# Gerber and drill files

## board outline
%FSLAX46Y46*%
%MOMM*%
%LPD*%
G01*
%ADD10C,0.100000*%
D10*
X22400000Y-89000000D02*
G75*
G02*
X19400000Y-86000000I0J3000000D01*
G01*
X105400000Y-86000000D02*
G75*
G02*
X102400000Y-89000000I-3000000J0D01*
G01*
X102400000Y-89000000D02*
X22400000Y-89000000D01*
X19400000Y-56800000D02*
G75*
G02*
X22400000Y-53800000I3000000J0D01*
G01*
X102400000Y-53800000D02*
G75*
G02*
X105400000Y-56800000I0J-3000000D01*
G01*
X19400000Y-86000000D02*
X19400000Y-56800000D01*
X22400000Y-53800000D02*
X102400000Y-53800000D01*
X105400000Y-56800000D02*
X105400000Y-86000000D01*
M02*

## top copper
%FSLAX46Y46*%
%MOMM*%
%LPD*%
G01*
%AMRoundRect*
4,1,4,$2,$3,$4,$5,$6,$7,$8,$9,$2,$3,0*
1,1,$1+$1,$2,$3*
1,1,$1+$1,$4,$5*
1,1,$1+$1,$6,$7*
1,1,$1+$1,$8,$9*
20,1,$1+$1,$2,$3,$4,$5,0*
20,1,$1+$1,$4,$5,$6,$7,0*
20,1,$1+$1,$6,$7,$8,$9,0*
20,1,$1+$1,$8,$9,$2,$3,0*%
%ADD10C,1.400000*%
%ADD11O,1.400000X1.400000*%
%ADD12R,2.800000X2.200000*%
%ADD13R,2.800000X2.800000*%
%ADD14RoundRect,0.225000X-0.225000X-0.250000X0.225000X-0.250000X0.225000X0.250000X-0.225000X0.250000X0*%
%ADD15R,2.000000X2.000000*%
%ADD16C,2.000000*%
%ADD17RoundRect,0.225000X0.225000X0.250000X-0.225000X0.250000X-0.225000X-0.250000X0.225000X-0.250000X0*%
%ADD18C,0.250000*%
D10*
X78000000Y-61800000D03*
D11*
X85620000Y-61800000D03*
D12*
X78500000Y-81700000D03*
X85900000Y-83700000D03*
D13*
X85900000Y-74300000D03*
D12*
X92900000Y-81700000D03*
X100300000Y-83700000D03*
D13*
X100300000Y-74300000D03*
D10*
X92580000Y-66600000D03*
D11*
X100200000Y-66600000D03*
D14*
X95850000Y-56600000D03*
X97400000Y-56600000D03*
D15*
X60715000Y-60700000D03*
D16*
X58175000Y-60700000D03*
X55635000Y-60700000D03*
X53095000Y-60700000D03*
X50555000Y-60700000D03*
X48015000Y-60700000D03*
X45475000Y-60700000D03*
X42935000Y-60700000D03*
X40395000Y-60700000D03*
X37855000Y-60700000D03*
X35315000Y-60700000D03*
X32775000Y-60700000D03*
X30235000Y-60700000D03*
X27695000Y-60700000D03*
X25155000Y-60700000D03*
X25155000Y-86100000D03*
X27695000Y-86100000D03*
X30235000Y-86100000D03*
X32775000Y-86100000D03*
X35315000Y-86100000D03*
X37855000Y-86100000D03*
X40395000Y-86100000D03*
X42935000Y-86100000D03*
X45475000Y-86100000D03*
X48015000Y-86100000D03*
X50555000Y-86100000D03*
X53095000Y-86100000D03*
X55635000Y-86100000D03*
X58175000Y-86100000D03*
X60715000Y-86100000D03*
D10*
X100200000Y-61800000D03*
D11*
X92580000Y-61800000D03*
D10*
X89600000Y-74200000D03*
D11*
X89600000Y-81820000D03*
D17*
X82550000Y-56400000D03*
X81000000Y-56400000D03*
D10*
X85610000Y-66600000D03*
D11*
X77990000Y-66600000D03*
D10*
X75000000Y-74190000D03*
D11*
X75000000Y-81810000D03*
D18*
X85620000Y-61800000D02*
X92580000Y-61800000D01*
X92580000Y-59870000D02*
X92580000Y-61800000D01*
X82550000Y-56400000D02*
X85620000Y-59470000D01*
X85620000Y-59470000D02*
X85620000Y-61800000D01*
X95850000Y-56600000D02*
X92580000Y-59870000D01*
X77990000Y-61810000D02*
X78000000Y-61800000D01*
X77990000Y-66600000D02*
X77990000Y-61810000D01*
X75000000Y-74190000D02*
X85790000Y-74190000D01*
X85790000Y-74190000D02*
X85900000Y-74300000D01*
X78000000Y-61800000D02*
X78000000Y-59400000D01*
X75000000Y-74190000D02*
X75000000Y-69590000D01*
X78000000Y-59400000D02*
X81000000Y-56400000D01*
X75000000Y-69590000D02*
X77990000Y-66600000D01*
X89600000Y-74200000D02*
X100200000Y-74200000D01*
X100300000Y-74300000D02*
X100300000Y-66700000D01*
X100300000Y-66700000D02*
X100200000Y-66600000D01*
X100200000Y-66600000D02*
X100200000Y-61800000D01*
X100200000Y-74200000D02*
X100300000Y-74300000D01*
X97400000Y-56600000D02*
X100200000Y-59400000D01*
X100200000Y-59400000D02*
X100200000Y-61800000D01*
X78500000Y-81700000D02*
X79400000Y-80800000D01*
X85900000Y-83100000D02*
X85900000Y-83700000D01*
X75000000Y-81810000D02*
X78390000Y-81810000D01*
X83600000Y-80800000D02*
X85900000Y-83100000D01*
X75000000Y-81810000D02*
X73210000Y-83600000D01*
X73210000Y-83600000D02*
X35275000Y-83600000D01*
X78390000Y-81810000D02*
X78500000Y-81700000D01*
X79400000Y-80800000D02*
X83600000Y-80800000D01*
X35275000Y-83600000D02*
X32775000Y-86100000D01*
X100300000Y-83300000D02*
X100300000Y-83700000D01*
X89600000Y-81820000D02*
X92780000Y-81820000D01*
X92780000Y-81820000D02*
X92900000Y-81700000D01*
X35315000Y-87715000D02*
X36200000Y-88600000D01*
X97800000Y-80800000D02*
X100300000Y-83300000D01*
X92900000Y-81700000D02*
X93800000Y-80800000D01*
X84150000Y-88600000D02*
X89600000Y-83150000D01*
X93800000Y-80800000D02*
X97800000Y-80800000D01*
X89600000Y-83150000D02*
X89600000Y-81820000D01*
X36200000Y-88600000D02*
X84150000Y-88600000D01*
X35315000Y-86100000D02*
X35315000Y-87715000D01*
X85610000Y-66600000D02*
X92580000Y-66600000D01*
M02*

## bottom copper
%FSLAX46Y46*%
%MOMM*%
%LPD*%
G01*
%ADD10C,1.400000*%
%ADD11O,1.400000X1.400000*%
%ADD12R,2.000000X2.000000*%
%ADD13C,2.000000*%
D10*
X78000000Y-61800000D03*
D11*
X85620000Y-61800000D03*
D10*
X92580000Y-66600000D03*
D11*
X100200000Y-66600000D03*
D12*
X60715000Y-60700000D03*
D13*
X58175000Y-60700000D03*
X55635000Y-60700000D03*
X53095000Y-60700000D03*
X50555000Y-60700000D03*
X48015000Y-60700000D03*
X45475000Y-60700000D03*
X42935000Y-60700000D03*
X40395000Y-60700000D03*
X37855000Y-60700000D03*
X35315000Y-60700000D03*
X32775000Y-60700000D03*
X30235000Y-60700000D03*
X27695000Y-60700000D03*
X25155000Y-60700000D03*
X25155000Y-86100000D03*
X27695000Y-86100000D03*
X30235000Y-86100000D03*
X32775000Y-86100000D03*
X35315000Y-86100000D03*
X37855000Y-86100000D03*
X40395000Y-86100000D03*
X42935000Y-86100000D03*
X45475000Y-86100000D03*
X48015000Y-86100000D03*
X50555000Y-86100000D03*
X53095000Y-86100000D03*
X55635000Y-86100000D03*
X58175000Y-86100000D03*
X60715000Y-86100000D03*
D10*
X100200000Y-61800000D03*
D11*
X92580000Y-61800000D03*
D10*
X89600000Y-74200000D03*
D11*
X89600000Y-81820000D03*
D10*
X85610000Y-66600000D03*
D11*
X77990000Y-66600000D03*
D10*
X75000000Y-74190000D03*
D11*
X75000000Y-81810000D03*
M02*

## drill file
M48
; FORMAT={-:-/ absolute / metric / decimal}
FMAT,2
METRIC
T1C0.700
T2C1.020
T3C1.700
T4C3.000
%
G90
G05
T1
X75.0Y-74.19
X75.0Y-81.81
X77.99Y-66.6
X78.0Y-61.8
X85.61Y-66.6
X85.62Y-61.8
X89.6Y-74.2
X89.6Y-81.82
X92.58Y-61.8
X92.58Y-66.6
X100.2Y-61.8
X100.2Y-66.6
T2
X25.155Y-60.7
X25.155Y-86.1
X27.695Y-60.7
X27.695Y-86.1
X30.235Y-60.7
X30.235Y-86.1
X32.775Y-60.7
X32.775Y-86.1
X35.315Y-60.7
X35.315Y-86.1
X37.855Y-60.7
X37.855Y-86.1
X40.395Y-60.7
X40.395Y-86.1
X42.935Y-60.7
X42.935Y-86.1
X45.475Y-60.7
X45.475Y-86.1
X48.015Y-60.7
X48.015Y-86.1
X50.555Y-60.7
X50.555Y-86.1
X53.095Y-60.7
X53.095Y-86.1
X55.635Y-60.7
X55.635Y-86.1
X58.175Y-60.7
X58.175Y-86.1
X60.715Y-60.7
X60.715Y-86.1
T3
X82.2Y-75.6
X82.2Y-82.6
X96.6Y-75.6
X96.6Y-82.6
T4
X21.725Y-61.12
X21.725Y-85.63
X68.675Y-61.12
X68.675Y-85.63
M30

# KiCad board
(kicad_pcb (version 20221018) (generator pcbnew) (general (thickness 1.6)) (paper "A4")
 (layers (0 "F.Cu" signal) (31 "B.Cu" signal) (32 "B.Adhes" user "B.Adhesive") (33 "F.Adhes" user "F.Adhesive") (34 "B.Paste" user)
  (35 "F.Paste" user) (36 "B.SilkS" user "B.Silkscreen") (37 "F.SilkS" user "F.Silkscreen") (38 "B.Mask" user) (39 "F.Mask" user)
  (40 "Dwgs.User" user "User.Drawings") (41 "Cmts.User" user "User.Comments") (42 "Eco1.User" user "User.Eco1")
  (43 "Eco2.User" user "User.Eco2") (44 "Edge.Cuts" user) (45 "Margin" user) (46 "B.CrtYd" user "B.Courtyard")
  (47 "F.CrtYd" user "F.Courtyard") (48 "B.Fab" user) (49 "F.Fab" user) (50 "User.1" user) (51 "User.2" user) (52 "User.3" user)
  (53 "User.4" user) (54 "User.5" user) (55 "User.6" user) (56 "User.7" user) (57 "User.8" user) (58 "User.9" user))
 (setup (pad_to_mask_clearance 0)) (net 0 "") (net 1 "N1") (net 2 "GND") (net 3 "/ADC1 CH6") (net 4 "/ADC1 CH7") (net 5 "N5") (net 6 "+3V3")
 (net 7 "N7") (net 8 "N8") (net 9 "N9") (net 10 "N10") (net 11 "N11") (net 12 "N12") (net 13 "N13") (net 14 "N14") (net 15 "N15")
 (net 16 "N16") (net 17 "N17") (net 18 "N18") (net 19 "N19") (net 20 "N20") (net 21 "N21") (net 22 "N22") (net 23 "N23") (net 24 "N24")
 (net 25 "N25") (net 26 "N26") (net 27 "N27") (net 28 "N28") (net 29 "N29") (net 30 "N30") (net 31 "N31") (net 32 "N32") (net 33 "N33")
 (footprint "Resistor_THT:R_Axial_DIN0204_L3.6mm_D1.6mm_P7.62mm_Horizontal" (layer "F.Cu") (at 78 61.8)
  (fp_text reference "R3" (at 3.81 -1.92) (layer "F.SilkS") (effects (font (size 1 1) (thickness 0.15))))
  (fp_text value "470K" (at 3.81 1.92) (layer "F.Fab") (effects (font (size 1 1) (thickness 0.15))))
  (pad "1" thru_hole circle (at 0 0) (size 1.4 1.4) (drill 0.7) (layers "*.Cu" "*.Mask") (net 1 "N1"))
  (pad "2" thru_hole oval (at 7.62 0) (size 1.4 1.4) (drill 0.7) (layers "*.Cu" "*.Mask") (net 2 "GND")))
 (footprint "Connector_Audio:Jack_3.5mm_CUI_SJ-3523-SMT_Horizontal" (layer "F.Cu") (at 82.2 80.1 180)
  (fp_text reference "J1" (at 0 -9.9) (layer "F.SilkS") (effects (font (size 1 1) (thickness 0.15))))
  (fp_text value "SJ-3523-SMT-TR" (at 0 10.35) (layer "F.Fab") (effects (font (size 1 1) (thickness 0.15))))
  (pad "" np_thru_hole circle (at 0 -2.5 180) (size 1.7 1.7) (drill 1.7) (layers "*.Cu" "*.Mask"))
  (pad "" np_thru_hole circle (at 0 4.5 180) (size 1.7 1.7) (drill 1.7) (layers "*.Cu" "*.Mask"))
  (pad "R" smd rect (at 3.7 -1.6 180) (size 2.8 2.2) (layers "F.Cu" "F.Paste" "F.Mask") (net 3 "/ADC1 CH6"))
  (pad "S" smd rect (at -3.7 -3.6 180) (size 2.8 2.2) (layers "F.Cu" "F.Paste" "F.Mask") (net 3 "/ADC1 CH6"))
  (pad "T" smd rect (at -3.7 5.8 180) (size 2.8 2.8) (layers "F.Cu" "F.Paste" "F.Mask") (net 1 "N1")))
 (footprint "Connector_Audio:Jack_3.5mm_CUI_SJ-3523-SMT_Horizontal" (layer "F.Cu") (at 96.6 80.1 180)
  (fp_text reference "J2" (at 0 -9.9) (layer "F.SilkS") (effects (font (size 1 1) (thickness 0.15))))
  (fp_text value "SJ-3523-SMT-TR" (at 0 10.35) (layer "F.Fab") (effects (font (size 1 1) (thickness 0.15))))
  (pad "" np_thru_hole circle (at 0 -2.5 180) (size 1.7 1.7) (drill 1.7) (layers "*.Cu" "*.Mask"))
  (pad "" np_thru_hole circle (at 0 4.5 180) (size 1.7 1.7) (drill 1.7) (layers "*.Cu" "*.Mask"))
  (pad "R" smd rect (at 3.7 -1.6 180) (size 2.8 2.2) (layers "F.Cu" "F.Paste" "F.Mask") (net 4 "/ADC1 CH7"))
  (pad "S" smd rect (at -3.7 -3.6 180) (size 2.8 2.2) (layers "F.Cu" "F.Paste" "F.Mask") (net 4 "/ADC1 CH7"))
  (pad "T" smd rect (at -3.7 5.8 180) (size 2.8 2.8) (layers "F.Cu" "F.Paste" "F.Mask") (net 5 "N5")))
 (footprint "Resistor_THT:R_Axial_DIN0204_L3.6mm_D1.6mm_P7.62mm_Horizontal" (layer "F.Cu") (at 92.58 66.6)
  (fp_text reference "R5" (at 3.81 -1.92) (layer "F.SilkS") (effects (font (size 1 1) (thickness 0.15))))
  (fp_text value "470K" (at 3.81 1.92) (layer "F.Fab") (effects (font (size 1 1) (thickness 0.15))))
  (pad "1" thru_hole circle (at 0 0) (size 1.4 1.4) (drill 0.7) (layers "*.Cu" "*.Mask") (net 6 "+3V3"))
  (pad "2" thru_hole oval (at 7.62 0) (size 1.4 1.4) (drill 0.7) (layers "*.Cu" "*.Mask") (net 5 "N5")))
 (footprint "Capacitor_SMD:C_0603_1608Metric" (layer "F.Cu") (at 96.625 56.6)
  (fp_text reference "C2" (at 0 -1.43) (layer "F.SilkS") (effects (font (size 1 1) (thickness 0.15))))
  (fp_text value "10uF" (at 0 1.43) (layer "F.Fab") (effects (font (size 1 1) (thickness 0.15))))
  (pad "1" smd roundrect (at -0.775 0) (size 0.9 0.95) (layers "F.Cu" "F.Paste" "F.Mask") (roundrect_rratio 0.25) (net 2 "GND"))
  (pad "2" smd roundrect (at 0.775 0) (size 0.9 0.95) (layers "F.Cu" "F.Paste" "F.Mask") (roundrect_rratio 0.25) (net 5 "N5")))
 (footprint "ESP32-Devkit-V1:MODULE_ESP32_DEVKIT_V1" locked (layer "F.Cu") (at 45.2 73.4 -90)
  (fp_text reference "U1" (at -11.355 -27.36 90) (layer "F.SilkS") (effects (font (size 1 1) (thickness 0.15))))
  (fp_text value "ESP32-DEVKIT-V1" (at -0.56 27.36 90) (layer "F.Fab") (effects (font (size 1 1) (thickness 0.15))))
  (pad "" np_thru_hole circle locked (at -12.28 -23.475 270) (size 3 3) (drill 3) (layers "*.Cu" "*.Mask"))
  (pad "" np_thru_hole circle locked (at -12.28 23.475 270) (size 3 3) (drill 3) (layers "*.Cu" "*.Mask"))
  (pad "" np_thru_hole circle locked (at 12.23 -23.475 270) (size 3 3) (drill 3) (layers "*.Cu" "*.Mask"))
  (pad "" np_thru_hole circle locked (at 12.23 23.475 270) (size 3 3) (drill 3) (layers "*.Cu" "*.Mask"))
  (pad "1" thru_hole rect locked (at -12.7 -15.515 270) (size 2 2) (drill 1.02) (layers "*.Cu" "*.Mask") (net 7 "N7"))
  (pad "2" thru_hole circle locked (at -12.7 -12.975 270) (size 2 2) (drill 1.02) (layers "*.Cu" "*.Mask") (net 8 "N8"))
  (pad "3" thru_hole circle locked (at -12.7 -10.435 270) (size 2 2) (drill 1.02) (layers "*.Cu" "*.Mask") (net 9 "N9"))
  (pad "4" thru_hole circle locked (at -12.7 -7.895 270) (size 2 2) (drill 1.02) (layers "*.Cu" "*.Mask") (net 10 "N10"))
  (pad "5" thru_hole circle locked (at -12.7 -5.355 270) (size 2 2) (drill 1.02) (layers "*.Cu" "*.Mask") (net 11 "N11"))
  (pad "6" thru_hole circle locked (at -12.7 -2.815 270) (size 2 2) (drill 1.02) (layers "*.Cu" "*.Mask") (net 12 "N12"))
  (pad "7" thru_hole circle locked (at -12.7 -0.275 270) (size 2 2) (drill 1.02) (layers "*.Cu" "*.Mask") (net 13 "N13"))
  (pad "8" thru_hole circle locked (at -12.7 2.265 270) (size 2 2) (drill 1.02) (layers "*.Cu" "*.Mask") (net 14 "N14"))
  (pad "9" thru_hole circle locked (at -12.7 4.805 270) (size 2 2) (drill 1.02) (layers "*.Cu" "*.Mask") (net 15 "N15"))
  (pad "10" thru_hole circle locked (at -12.7 7.345 270) (size 2 2) (drill 1.02) (layers "*.Cu" "*.Mask") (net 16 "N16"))
  (pad "11" thru_hole circle locked (at -12.7 9.885 270) (size 2 2) (drill 1.02) (layers "*.Cu" "*.Mask") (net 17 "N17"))
  (pad "12" thru_hole circle locked (at -12.7 12.425 270) (size 2 2) (drill 1.02) (layers "*.Cu" "*.Mask") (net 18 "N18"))
  (pad "13" thru_hole circle locked (at -12.7 14.965 270) (size 2 2) (drill 1.02) (layers "*.Cu" "*.Mask") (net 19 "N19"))
  (pad "14" thru_hole circle locked (at -12.7 17.505 270) (size 2 2) (drill 1.02) (layers "*.Cu" "*.Mask") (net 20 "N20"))
  (pad "15" thru_hole circle locked (at -12.7 20.045 270) (size 2 2) (drill 1.02) (layers "*.Cu" "*.Mask") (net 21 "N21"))
  (pad "16" thru_hole circle locked (at 12.7 20.045 270) (size 2 2) (drill 1.02) (layers "*.Cu" "*.Mask") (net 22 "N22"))
  (pad "17" thru_hole circle locked (at 12.7 17.505 270) (size 2 2) (drill 1.02) (layers "*.Cu" "*.Mask") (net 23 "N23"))
  (pad "18" thru_hole circle locked (at 12.7 14.965 270) (size 2 2) (drill 1.02) (layers "*.Cu" "*.Mask") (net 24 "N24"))
  (pad "19" thru_hole circle locked (at 12.7 12.425 270) (size 2 2) (drill 1.02) (layers "*.Cu" "*.Mask") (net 3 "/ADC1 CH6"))
  (pad "20" thru_hole circle locked (at 12.7 9.885 270) (size 2 2) (drill 1.02) (layers "*.Cu" "*.Mask") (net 4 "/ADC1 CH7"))
  (pad "21" thru_hole circle locked (at 12.7 7.345 270) (size 2 2) (drill 1.02) (layers "*.Cu" "*.Mask") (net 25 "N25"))
  (pad "22" thru_hole circle locked (at 12.7 4.805 270) (size 2 2) (drill 1.02) (layers "*.Cu" "*.Mask") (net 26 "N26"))
  (pad "23" thru_hole circle locked (at 12.7 2.265 270) (size 2 2) (drill 1.02) (layers "*.Cu" "*.Mask") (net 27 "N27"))
  (pad "24" thru_hole circle locked (at 12.7 -0.275 270) (size 2 2) (drill 1.02) (layers "*.Cu" "*.Mask") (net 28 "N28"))
  (pad "25" thru_hole circle locked (at 12.7 -2.815 270) (size 2 2) (drill 1.02) (layers "*.Cu" "*.Mask") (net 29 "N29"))
  (pad "26" thru_hole circle locked (at 12.7 -5.355 270) (size 2 2) (drill 1.02) (layers "*.Cu" "*.Mask") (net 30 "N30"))
  (pad "27" thru_hole circle locked (at 12.7 -7.895 270) (size 2 2) (drill 1.02) (layers "*.Cu" "*.Mask") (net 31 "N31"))
  (pad "28" thru_hole circle locked (at 12.7 -10.435 270) (size 2 2) (drill 1.02) (layers "*.Cu" "*.Mask") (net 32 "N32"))
  (pad "29" thru_hole circle locked (at 12.7 -12.975 270) (size 2 2) (drill 1.02) (layers "*.Cu" "*.Mask") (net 8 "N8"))
  (pad "30" thru_hole circle locked (at 12.7 -15.515 270) (size 2 2) (drill 1.02) (layers "*.Cu" "*.Mask") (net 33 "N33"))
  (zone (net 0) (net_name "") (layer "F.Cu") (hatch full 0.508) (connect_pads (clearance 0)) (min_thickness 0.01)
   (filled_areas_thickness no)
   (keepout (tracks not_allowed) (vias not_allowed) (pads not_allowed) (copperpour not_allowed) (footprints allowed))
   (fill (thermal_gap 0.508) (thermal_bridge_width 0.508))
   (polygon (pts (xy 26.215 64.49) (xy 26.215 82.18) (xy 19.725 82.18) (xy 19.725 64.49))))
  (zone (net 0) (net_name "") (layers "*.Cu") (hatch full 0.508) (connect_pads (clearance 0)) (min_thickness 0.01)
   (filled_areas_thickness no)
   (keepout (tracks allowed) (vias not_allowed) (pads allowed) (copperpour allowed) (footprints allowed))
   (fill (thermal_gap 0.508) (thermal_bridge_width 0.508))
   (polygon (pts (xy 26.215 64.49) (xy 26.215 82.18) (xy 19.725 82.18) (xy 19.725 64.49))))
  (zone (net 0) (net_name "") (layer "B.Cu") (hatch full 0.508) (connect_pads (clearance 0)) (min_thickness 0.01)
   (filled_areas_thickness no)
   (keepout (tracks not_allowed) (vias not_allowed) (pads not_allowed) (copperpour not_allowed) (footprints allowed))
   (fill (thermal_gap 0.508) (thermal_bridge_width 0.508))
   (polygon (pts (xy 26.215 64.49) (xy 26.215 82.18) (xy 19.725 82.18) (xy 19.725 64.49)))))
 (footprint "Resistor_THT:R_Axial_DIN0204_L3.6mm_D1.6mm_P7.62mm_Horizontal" (layer "F.Cu") (at 100.2 61.8 180)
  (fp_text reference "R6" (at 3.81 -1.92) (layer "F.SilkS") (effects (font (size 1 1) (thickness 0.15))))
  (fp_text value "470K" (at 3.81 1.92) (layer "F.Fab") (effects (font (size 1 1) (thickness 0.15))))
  (pad "1" thru_hole circle (at 0 0 180) (size 1.4 1.4) (drill 0.7) (layers "*.Cu" "*.Mask") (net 5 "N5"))
  (pad "2" thru_hole oval (at 7.62 0 180) (size 1.4 1.4) (drill 0.7) (layers "*.Cu" "*.Mask") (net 2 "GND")))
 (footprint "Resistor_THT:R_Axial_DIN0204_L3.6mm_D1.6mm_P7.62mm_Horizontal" (layer "F.Cu") (at 89.6 74.2 -90)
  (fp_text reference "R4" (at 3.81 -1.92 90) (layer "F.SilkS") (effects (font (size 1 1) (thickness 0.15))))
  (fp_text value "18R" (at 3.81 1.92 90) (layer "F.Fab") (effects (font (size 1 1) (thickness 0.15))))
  (pad "1" thru_hole circle (at 0 0 270) (size 1.4 1.4) (drill 0.7) (layers "*.Cu" "*.Mask") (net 5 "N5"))
  (pad "2" thru_hole oval (at 7.62 0 270) (size 1.4 1.4) (drill 0.7) (layers "*.Cu" "*.Mask") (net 4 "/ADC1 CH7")))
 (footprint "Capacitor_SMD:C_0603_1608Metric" (layer "F.Cu") (at 81.775 56.4 180)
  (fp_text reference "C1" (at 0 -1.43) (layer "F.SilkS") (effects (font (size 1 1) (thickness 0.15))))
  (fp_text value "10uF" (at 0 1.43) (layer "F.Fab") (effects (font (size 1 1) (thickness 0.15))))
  (pad "1" smd roundrect (at -0.775 0 180) (size 0.9 0.95) (layers "F.Cu" "F.Paste" "F.Mask") (roundrect_rratio 0.25) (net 2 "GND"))
  (pad "2" smd roundrect (at 0.775 0 180) (size 0.9 0.95) (layers "F.Cu" "F.Paste" "F.Mask") (roundrect_rratio 0.25) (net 1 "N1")))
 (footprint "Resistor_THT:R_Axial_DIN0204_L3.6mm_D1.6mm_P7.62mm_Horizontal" (layer "F.Cu") (at 85.61 66.6 180)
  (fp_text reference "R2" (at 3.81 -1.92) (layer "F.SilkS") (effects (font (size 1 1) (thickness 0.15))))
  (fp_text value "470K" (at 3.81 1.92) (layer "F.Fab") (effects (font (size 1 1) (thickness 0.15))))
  (pad "1" thru_hole circle (at 0 0 180) (size 1.4 1.4) (drill 0.7) (layers "*.Cu" "*.Mask") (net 6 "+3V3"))
  (pad "2" thru_hole oval (at 7.62 0 180) (size 1.4 1.4) (drill 0.7) (layers "*.Cu" "*.Mask") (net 1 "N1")))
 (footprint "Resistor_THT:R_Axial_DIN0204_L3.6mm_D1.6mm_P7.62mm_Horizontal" (layer "F.Cu") (at 75 74.19 -90)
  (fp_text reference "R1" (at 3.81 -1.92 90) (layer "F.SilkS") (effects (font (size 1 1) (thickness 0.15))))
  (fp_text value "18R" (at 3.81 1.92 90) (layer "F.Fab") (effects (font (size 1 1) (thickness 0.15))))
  (pad "1" thru_hole circle (at 0 0 270) (size 1.4 1.4) (drill 0.7) (layers "*.Cu" "*.Mask") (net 1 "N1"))
  (pad "2" thru_hole oval (at 7.62 0 270) (size 1.4 1.4) (drill 0.7) (layers "*.Cu" "*.Mask") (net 3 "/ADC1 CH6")))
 (gr_arc (start 22.4 89) (mid 20.27868 88.12132) (end 19.4 86) (stroke (width 0.1) (type default)) (layer "Edge.Cuts"))
 (gr_arc (start 105.4 86) (mid 104.52132 88.12132) (end 102.4 89) (stroke (width 0.1) (type default)) (layer "Edge.Cuts"))
 (gr_line (start 102.4 89) (end 22.4 89) (stroke (width 0.1) (type default)) (layer "Edge.Cuts"))
 (gr_arc (start 19.4 56.8) (mid 20.27868 54.67868) (end 22.4 53.8) (stroke (width 0.1) (type default)) (layer "Edge.Cuts"))
 (gr_arc (start 102.4 53.8) (mid 104.52132 54.67868) (end 105.4 56.8) (stroke (width 0.1) (type default)) (layer "Edge.Cuts"))
 (gr_line (start 19.4 86) (end 19.4 56.8) (stroke (width 0.1) (type default)) (layer "Edge.Cuts"))
 (gr_line (start 22.4 53.8) (end 102.4 53.8) (stroke (width 0.1) (type default)) (layer "Edge.Cuts"))
 (gr_line (start 105.4 56.8) (end 105.4 86) (stroke (width 0.1) (type default)) (layer "Edge.Cuts"))
 (segment (start 85.62 61.8) (end 92.58 61.8) (width 0.25) (layer "F.Cu") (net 2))
 (segment (start 92.58 59.87) (end 92.58 61.8) (width 0.25) (layer "F.Cu") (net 2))
 (segment (start 82.55 56.4) (end 85.62 59.47) (width 0.25) (layer "F.Cu") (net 2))
 (segment (start 85.62 59.47) (end 85.62 61.8) (width 0.25) (layer "F.Cu") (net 2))
 (segment (start 95.85 56.6) (end 92.58 59.87) (width 0.25) (layer "F.Cu") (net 2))
 (segment (start 77.99 61.81) (end 78 61.8) (width 0.25) (layer "F.Cu") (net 1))
 (segment (start 77.99 66.6) (end 77.99 61.81) (width 0.25) (layer "F.Cu") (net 1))
 (segment (start 75 74.19) (end 85.79 74.19) (width 0.25) (layer "F.Cu") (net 1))
 (segment (start 85.79 74.19) (end 85.9 74.3) (width 0.25) (layer "F.Cu") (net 1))
 (segment (start 78 61.8) (end 78 59.4) (width 0.25) (layer "F.Cu") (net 1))
 (segment (start 75 74.19) (end 75 69.59) (width 0.25) (layer "F.Cu") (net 1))
 (segment (start 78 59.4) (end 81 56.4) (width 0.25) (layer "F.Cu") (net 1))
 (segment (start 75 69.59) (end 77.99 66.6) (width 0.25) (layer "F.Cu") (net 1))
 (segment (start 89.6 74.2) (end 100.2 74.2) (width 0.25) (layer "F.Cu") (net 5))
 (segment (start 100.3 74.3) (end 100.3 66.7) (width 0.25) (layer "F.Cu") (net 5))
 (segment (start 100.3 66.7) (end 100.2 66.6) (width 0.25) (layer "F.Cu") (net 5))
 (segment (start 100.2 66.6) (end 100.2 61.8) (width 0.25) (layer "F.Cu") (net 5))
 (segment (start 100.2 74.2) (end 100.3 74.3) (width 0.25) (layer "F.Cu") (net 5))
 (segment (start 97.4 56.6) (end 100.2 59.4) (width 0.25) (layer "F.Cu") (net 5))
 (segment (start 100.2 59.4) (end 100.2 61.8) (width 0.25) (layer "F.Cu") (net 5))
 (segment (start 78.5 81.7) (end 79.4 80.8) (width 0.25) (layer "F.Cu") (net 3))
 (segment (start 85.9 83.1) (end 85.9 83.7) (width 0.25) (layer "F.Cu") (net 3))
 (segment (start 75 81.81) (end 78.39 81.81) (width 0.25) (layer "F.Cu") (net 3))
 (segment (start 83.6 80.8) (end 85.9 83.1) (width 0.25) (layer "F.Cu") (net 3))
 (segment (start 75 81.81) (end 73.21 83.6) (width 0.25) (layer "F.Cu") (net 3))
 (segment (start 73.21 83.6) (end 35.275 83.6) (width 0.25) (layer "F.Cu") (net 3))
 (segment (start 78.39 81.81) (end 78.5 81.7) (width 0.25) (layer "F.Cu") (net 3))
 (segment (start 79.4 80.8) (end 83.6 80.8) (width 0.25) (layer "F.Cu") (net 3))
 (segment (start 35.275 83.6) (end 32.775 86.1) (width 0.25) (layer "F.Cu") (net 3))
 (segment (start 100.3 83.3) (end 100.3 83.7) (width 0.25) (layer "F.Cu") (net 4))
 (segment (start 89.6 81.82) (end 92.78 81.82) (width 0.25) (layer "F.Cu") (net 4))
 (segment (start 92.78 81.82) (end 92.9 81.7) (width 0.25) (layer "F.Cu") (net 4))
 (segment (start 35.315 87.715) (end 36.2 88.6) (width 0.25) (layer "F.Cu") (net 4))
 (segment (start 97.8 80.8) (end 100.3 83.3) (width 0.25) (layer "F.Cu") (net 4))
 (segment (start 92.9 81.7) (end 93.8 80.8) (width 0.25) (layer "F.Cu") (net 4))
 (segment (start 84.15 88.6) (end 89.6 83.15) (width 0.25) (layer "F.Cu") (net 4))
 (segment (start 93.8 80.8) (end 97.8 80.8) (width 0.25) (layer "F.Cu") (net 4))
 (segment (start 89.6 83.15) (end 89.6 81.82) (width 0.25) (layer "F.Cu") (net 4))
 (segment (start 36.2 88.6) (end 84.15 88.6) (width 0.25) (layer "F.Cu") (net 4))
 (segment (start 35.315 86.1) (end 35.315 87.715) (width 0.25) (layer "F.Cu") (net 4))
 (segment (start 85.61 66.6) (end 92.58 66.6) (width 0.25) (layer "F.Cu") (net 6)))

